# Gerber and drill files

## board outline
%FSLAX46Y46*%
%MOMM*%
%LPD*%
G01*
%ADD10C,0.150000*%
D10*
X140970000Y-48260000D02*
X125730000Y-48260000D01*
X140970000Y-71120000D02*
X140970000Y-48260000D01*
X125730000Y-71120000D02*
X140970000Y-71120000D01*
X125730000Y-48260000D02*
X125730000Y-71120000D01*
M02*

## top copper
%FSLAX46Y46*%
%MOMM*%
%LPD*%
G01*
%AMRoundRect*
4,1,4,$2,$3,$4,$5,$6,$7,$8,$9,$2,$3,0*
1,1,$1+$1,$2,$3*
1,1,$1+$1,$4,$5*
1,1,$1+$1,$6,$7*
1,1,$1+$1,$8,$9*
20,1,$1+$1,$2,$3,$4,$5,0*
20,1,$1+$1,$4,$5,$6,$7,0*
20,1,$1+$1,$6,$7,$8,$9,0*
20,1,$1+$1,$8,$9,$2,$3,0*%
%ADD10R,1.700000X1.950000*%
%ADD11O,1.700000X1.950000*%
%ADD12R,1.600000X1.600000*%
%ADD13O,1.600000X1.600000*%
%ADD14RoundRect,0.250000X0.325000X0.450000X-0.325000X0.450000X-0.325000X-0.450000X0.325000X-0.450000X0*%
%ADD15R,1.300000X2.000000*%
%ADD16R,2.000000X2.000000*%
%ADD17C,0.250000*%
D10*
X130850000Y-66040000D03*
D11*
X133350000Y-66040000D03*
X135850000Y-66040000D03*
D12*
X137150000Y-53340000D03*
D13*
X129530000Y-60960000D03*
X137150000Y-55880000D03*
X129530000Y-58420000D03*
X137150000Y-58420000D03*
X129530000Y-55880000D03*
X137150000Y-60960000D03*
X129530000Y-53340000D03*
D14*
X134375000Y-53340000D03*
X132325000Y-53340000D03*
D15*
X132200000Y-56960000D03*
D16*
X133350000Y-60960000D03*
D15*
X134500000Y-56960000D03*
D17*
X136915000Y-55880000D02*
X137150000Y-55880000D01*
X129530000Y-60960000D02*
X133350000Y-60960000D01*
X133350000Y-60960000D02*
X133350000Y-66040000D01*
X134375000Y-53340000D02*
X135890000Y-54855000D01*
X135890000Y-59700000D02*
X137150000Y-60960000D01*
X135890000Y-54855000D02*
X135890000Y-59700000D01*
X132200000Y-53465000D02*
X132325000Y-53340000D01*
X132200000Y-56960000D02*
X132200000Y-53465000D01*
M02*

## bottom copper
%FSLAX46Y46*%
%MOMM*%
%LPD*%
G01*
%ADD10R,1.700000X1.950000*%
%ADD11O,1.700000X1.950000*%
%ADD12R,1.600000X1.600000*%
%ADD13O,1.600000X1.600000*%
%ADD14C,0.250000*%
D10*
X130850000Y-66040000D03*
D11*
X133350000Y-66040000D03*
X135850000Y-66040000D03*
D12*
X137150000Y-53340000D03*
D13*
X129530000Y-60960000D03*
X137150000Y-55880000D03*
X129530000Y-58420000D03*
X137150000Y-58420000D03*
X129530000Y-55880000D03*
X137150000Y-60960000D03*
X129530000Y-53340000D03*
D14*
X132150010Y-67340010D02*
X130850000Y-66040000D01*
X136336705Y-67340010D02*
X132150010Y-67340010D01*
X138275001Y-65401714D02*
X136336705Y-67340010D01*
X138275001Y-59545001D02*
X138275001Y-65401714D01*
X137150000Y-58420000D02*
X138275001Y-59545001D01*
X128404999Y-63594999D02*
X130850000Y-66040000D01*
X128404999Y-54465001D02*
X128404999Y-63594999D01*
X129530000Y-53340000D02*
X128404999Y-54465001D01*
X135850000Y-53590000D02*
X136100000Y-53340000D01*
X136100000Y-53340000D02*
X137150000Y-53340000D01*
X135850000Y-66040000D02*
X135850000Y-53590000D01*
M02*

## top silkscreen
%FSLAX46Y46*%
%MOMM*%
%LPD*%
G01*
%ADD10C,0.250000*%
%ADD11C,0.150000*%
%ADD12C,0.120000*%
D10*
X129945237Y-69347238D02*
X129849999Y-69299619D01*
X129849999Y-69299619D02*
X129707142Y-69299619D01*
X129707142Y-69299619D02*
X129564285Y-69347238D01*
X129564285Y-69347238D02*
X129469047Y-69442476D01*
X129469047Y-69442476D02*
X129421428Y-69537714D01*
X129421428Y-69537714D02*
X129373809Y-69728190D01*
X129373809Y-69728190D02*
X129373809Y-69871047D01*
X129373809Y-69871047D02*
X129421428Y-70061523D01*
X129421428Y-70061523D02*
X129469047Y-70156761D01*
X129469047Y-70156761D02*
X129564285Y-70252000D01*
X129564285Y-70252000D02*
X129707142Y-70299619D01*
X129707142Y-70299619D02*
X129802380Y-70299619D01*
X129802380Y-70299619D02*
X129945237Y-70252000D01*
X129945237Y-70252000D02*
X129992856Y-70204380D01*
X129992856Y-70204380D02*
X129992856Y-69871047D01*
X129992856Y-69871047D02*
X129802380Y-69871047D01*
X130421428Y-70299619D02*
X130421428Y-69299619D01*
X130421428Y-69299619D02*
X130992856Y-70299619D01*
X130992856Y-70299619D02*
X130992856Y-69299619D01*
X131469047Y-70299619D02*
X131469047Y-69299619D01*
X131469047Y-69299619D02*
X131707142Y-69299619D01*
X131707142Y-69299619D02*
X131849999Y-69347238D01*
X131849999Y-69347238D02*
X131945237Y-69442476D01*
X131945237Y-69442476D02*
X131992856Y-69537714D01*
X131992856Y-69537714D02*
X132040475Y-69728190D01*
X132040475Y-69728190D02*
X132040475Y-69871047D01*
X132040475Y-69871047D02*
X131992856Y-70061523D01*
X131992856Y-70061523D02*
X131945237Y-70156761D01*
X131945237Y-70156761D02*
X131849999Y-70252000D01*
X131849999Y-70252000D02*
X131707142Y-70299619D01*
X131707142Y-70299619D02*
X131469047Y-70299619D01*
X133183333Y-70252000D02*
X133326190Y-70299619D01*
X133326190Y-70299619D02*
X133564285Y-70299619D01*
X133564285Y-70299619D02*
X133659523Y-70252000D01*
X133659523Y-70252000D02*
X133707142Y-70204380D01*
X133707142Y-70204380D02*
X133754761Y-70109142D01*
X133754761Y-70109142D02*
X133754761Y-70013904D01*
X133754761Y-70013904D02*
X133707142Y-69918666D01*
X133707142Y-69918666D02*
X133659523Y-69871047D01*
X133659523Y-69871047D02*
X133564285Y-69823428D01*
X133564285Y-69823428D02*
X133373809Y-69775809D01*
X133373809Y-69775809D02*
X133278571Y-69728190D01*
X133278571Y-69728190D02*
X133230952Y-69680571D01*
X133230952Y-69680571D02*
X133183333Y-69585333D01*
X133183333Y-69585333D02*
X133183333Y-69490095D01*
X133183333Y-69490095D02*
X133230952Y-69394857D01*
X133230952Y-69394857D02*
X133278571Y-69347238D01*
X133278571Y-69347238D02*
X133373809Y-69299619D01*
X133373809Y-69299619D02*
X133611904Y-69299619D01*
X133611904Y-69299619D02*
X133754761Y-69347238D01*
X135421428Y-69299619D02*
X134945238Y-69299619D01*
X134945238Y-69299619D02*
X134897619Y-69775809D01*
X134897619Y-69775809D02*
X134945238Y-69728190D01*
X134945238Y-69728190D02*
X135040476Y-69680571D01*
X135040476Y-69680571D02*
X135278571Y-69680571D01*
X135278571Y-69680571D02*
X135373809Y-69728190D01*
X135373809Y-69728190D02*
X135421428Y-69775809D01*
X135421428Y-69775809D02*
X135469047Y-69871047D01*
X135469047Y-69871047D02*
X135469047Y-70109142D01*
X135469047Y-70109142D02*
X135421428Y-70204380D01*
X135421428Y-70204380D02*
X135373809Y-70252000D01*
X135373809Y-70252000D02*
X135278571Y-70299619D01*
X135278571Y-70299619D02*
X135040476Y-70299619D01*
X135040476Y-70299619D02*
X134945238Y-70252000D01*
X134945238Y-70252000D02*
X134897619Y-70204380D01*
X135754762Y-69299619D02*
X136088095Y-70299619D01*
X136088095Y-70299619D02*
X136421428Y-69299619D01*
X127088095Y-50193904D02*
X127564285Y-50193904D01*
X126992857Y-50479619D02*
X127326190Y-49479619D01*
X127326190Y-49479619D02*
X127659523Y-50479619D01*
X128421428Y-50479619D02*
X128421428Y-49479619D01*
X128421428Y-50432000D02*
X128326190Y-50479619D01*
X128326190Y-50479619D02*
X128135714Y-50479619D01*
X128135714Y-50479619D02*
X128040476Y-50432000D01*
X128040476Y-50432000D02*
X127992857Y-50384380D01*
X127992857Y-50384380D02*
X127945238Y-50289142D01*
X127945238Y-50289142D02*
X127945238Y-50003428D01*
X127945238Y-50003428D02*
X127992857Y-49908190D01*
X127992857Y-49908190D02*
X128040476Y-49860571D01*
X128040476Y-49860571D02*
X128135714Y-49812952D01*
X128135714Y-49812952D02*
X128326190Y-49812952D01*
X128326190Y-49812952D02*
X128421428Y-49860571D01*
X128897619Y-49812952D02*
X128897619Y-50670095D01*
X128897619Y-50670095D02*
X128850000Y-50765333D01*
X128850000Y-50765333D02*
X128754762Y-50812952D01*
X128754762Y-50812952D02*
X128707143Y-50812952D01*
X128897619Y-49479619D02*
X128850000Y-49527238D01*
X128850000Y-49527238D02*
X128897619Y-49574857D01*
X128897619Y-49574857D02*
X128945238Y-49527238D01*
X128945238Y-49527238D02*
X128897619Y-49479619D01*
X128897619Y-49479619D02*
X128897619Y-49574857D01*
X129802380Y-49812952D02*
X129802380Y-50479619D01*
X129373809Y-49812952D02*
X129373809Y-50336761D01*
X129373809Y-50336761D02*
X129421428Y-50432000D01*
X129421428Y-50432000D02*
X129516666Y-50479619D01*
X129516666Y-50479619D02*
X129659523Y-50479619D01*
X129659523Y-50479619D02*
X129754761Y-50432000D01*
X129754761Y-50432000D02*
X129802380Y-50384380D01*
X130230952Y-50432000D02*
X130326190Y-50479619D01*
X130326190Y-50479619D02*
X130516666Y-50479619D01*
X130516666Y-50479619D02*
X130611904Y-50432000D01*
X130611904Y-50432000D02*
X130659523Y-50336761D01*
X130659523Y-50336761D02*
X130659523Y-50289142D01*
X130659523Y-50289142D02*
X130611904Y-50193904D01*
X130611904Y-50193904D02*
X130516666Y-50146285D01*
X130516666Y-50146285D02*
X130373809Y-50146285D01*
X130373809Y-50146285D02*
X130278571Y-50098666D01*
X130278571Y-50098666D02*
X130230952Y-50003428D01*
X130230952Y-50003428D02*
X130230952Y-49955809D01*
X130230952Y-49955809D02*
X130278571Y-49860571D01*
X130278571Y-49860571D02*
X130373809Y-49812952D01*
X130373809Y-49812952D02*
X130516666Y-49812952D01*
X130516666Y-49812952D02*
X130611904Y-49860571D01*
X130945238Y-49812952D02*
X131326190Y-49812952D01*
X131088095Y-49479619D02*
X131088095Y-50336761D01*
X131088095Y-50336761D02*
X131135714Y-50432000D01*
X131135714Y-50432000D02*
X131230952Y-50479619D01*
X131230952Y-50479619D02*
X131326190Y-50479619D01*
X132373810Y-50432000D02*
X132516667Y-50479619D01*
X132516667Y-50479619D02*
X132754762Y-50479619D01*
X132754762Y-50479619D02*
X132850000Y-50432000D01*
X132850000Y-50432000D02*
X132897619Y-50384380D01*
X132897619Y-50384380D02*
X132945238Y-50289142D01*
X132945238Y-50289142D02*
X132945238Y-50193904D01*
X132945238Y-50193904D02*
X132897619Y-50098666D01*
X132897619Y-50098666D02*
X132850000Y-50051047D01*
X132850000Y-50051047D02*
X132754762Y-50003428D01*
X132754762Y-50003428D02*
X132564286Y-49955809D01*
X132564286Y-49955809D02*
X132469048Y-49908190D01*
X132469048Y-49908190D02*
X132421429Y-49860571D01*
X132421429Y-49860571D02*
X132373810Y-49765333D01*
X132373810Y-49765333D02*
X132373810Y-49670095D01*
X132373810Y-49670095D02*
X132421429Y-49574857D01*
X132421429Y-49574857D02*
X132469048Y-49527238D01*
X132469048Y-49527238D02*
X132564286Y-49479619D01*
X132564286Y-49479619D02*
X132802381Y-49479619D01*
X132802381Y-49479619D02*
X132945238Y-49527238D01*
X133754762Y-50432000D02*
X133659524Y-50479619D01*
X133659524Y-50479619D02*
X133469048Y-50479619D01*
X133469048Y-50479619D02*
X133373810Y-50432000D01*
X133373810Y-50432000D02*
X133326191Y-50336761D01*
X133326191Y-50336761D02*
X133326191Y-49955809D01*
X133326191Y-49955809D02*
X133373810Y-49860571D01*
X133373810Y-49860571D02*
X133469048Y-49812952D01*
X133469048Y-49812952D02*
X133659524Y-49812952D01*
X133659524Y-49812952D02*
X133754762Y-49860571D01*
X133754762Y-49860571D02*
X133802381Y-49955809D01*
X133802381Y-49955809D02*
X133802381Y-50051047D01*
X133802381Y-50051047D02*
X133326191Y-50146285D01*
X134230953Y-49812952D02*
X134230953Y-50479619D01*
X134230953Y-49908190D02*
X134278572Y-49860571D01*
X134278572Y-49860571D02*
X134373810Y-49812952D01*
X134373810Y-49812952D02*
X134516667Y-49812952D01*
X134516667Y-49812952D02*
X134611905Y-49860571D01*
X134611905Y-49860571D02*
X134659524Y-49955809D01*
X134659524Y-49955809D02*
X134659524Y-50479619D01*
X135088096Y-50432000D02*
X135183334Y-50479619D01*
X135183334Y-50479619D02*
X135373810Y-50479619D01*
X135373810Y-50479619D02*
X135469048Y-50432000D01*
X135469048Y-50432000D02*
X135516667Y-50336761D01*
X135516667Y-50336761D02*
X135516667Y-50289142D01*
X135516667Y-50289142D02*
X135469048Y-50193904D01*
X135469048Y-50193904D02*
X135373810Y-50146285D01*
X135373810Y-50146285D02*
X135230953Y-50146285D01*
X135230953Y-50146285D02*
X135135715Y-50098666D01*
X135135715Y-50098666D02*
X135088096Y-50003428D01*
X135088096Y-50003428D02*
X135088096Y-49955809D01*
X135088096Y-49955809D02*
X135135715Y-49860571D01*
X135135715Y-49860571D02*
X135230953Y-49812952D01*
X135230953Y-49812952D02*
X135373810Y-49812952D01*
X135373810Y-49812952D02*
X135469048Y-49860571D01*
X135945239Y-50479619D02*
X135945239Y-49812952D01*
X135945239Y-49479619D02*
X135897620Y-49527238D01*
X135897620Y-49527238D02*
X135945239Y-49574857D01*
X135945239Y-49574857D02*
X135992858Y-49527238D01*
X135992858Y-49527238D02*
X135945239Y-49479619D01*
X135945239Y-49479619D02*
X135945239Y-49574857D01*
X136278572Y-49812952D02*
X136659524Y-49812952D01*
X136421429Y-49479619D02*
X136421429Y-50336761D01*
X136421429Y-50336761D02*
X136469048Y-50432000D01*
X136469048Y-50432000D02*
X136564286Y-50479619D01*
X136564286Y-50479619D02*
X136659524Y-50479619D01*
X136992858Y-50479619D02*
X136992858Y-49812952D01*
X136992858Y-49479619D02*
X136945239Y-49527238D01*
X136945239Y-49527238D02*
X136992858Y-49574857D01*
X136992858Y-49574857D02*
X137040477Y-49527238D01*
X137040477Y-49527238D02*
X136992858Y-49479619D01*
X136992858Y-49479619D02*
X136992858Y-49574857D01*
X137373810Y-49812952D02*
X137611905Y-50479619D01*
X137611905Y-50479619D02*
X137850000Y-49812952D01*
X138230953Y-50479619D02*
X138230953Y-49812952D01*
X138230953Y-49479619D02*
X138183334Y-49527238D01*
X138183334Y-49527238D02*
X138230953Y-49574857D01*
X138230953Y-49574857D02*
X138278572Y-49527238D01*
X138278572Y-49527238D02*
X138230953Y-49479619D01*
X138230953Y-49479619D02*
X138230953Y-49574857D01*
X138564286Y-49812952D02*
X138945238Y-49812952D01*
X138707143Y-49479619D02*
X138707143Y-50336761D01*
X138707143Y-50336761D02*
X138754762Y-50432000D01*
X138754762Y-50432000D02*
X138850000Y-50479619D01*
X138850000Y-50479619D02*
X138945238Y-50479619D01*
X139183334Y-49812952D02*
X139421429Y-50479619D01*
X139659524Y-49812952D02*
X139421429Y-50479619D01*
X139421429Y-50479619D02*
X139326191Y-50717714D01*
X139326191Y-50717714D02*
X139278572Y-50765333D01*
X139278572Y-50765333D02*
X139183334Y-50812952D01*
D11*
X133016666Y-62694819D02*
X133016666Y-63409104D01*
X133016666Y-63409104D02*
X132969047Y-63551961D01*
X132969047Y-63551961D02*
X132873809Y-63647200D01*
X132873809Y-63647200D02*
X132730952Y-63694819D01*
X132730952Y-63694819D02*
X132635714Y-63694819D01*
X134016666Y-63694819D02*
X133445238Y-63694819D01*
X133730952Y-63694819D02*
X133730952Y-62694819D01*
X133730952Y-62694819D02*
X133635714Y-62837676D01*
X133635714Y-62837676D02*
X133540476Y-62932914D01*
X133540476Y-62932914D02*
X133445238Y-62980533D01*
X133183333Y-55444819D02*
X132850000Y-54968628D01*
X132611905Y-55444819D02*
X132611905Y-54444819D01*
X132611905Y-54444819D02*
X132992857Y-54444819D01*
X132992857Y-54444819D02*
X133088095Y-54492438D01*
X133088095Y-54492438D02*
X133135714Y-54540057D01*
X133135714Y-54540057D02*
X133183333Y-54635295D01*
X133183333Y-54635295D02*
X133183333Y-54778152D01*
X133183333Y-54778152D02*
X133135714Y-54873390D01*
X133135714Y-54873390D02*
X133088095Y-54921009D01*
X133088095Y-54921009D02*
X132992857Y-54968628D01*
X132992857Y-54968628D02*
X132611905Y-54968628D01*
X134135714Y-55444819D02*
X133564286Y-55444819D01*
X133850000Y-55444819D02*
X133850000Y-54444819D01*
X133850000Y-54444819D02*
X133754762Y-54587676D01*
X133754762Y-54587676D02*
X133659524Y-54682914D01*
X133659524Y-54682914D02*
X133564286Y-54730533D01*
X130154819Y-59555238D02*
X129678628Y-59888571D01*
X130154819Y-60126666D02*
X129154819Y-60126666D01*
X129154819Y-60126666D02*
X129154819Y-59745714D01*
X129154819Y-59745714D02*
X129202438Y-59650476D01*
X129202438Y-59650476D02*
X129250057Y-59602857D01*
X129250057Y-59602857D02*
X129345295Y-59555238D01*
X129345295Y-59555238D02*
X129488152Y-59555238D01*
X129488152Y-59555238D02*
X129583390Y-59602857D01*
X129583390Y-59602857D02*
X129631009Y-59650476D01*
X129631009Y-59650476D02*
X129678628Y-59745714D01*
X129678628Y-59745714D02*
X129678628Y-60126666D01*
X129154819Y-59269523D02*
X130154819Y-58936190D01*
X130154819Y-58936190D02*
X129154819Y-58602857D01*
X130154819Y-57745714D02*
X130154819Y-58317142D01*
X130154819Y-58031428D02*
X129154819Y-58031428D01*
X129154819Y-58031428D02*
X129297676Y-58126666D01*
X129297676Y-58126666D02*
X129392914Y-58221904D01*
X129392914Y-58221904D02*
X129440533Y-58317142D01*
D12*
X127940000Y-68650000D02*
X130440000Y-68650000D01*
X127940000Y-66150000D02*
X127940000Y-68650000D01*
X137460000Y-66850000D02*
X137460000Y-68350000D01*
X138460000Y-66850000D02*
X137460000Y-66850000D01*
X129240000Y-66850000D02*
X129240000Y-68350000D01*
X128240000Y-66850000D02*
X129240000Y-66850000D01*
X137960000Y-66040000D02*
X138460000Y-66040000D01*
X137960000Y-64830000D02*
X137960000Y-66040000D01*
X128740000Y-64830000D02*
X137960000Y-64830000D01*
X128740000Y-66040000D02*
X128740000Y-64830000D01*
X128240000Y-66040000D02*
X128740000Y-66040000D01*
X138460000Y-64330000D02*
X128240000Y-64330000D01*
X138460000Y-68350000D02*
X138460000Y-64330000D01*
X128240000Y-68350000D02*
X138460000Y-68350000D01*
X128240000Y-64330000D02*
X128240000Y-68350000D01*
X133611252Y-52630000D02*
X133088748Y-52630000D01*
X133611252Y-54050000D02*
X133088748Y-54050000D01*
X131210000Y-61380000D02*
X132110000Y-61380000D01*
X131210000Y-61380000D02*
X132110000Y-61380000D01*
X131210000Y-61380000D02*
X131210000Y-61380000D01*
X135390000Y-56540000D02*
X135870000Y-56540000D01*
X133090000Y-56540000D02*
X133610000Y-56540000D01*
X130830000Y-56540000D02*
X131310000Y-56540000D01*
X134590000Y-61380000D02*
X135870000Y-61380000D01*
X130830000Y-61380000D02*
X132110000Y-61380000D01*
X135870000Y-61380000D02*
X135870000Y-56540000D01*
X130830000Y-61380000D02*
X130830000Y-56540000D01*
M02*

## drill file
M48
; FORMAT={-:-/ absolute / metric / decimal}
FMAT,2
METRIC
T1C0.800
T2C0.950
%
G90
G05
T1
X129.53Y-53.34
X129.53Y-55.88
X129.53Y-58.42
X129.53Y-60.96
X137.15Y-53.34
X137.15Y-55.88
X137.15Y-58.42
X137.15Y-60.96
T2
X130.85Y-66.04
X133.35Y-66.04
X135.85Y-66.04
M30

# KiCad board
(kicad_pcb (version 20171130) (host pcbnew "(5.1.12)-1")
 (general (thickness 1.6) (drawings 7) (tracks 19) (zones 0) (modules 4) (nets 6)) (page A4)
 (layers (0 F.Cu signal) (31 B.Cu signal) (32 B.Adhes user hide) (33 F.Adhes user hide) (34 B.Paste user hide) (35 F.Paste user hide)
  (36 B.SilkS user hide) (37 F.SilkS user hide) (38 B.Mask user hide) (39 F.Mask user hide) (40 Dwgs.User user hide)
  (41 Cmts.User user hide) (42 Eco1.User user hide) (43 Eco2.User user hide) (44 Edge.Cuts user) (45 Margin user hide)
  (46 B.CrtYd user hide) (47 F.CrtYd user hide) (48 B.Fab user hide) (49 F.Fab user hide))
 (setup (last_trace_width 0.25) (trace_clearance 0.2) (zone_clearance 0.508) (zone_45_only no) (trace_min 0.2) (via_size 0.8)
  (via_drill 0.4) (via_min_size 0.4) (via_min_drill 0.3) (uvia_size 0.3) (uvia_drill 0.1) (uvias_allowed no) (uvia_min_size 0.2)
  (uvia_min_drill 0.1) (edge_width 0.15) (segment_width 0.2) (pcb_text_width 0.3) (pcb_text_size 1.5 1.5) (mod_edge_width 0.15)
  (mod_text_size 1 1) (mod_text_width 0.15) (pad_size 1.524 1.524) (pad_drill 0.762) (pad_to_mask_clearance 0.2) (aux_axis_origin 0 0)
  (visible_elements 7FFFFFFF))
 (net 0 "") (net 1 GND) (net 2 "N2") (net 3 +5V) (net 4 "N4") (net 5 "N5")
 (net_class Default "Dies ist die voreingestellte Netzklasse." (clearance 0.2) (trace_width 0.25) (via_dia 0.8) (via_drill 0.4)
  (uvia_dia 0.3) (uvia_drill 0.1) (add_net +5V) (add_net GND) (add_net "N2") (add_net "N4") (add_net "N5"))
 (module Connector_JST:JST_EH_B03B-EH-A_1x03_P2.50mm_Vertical (layer F.Cu) (at 130.85 66.04)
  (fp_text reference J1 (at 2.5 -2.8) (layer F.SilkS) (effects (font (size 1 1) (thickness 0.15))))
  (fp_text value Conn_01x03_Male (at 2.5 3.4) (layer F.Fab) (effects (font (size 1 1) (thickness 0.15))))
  (fp_line (start -2.91 2.61) (end -0.41 2.61) (layer F.SilkS) (width 0.12))
  (fp_line (start -2.91 0.11) (end -2.91 2.61) (layer F.SilkS) (width 0.12))
  (fp_line (start 6.61 0.81) (end 6.61 2.31) (layer F.SilkS) (width 0.12))
  (fp_line (start 7.61 0.81) (end 6.61 0.81) (layer F.SilkS) (width 0.12))
  (fp_line (start -1.61 0.81) (end -1.61 2.31) (layer F.SilkS) (width 0.12))
  (fp_line (start -2.61 0.81) (end -1.61 0.81) (layer F.SilkS) (width 0.12))
  (fp_line (start 7.11 0) (end 7.61 0) (layer F.SilkS) (width 0.12))
  (fp_line (start 7.11 -1.21) (end 7.11 0) (layer F.SilkS) (width 0.12))
  (fp_line (start -2.11 -1.21) (end 7.11 -1.21) (layer F.SilkS) (width 0.12))
  (fp_line (start -2.11 0) (end -2.11 -1.21) (layer F.SilkS) (width 0.12))
  (fp_line (start -2.61 0) (end -2.11 0) (layer F.SilkS) (width 0.12))
  (fp_line (start 7.61 -1.71) (end -2.61 -1.71) (layer F.SilkS) (width 0.12))
  (fp_line (start 7.61 2.31) (end 7.61 -1.71) (layer F.SilkS) (width 0.12))
  (fp_line (start -2.61 2.31) (end 7.61 2.31) (layer F.SilkS) (width 0.12))
  (fp_line (start -2.61 -1.71) (end -2.61 2.31) (layer F.SilkS) (width 0.12))
  (pad 1 thru_hole rect (at 0 0) (size 1.7 1.95) (drill 0.95) (layers *.Cu *.Mask) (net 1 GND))
  (pad 2 thru_hole oval (at 2.5 0) (size 1.7 1.95) (drill 0.95) (layers *.Cu *.Mask) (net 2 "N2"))
  (pad 3 thru_hole oval (at 5 0) (size 1.7 1.95) (drill 0.95) (layers *.Cu *.Mask) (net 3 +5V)))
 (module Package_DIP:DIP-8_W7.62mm (layer B.Cu) (at 137.15 53.34 180)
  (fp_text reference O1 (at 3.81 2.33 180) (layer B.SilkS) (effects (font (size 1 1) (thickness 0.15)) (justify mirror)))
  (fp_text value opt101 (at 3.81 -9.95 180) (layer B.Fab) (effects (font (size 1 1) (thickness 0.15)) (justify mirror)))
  (pad 1 thru_hole rect (at 0 0 180) (size 1.6 1.6) (drill 0.8) (layers *.Cu *.Mask) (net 3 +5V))
  (pad 5 thru_hole oval (at 7.62 -7.62 180) (size 1.6 1.6) (drill 0.8) (layers *.Cu *.Mask) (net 2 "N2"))
  (pad 2 thru_hole oval (at 0 -2.54 180) (size 1.6 1.6) (drill 0.8) (layers *.Cu *.Mask))
  (pad 6 thru_hole oval (at 7.62 -5.08 180) (size 1.6 1.6) (drill 0.8) (layers *.Cu *.Mask))
  (pad 3 thru_hole oval (at 0 -5.08 180) (size 1.6 1.6) (drill 0.8) (layers *.Cu *.Mask) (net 1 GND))
  (pad 7 thru_hole oval (at 7.62 -2.54 180) (size 1.6 1.6) (drill 0.8) (layers *.Cu *.Mask))
  (pad 4 thru_hole oval (at 0 -7.62 180) (size 1.6 1.6) (drill 0.8) (layers *.Cu *.Mask) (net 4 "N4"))
  (pad 8 thru_hole oval (at 7.62 0 180) (size 1.6 1.6) (drill 0.8) (layers *.Cu *.Mask) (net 1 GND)))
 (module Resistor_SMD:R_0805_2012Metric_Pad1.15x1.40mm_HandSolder (layer F.Cu) (at 133.35 53.34 180)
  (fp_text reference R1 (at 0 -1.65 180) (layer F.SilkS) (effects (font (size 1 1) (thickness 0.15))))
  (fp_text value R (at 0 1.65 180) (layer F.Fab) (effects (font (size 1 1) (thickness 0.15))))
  (fp_line (start -0.261252 0.71) (end 0.261252 0.71) (layer F.SilkS) (width 0.12))
  (fp_line (start -0.261252 -0.71) (end 0.261252 -0.71) (layer F.SilkS) (width 0.12))
  (pad 1 smd roundrect (at -1.025 0 180) (size 1.15 1.4) (layers F.Cu F.Paste F.Mask) (roundrect_rratio 0.217391) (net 4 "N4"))
  (pad 2 smd roundrect (at 1.025 0 180) (size 1.15 1.4) (layers F.Cu F.Paste F.Mask) (roundrect_rratio 0.217391) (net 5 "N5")))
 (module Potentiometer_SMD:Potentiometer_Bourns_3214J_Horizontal (layer F.Cu) (at 133.35 58.96 90)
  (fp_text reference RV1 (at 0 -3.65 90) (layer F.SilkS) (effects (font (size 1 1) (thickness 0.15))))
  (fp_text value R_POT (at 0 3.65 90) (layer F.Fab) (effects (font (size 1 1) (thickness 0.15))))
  (fp_line (start -2.42 -2.14) (end -2.42 -1.24) (layer F.SilkS) (width 0.12))
  (fp_line (start -2.42 -2.14) (end -2.42 -1.24) (layer F.SilkS) (width 0.12))
  (fp_line (start -2.42 -2.14) (end -2.42 -2.14) (layer F.SilkS) (width 0.12))
  (fp_line (start 2.42 2.04) (end 2.42 2.52) (layer F.SilkS) (width 0.12))
  (fp_line (start 2.42 -0.26) (end 2.42 0.26) (layer F.SilkS) (width 0.12))
  (fp_line (start 2.42 -2.52) (end 2.42 -2.04) (layer F.SilkS) (width 0.12))
  (fp_line (start -2.42 1.24) (end -2.42 2.52) (layer F.SilkS) (width 0.12))
  (fp_line (start -2.42 -2.52) (end -2.42 -1.24) (layer F.SilkS) (width 0.12))
  (fp_line (start -2.42 2.52) (end 2.42 2.52) (layer F.SilkS) (width 0.12))
  (fp_line (start -2.42 -2.52) (end 2.42 -2.52) (layer F.SilkS) (width 0.12))
  (pad 1 smd rect (at 2 -1.15 90) (size 2 1.3) (layers F.Cu F.Paste F.Mask) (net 5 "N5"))
  (pad 2 smd rect (at -2 0 90) (size 2 2) (layers F.Cu F.Paste F.Mask) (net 2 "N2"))
  (pad 3 smd rect (at 2 1.15 90) (size 2 1.3) (layers F.Cu F.Paste F.Mask)))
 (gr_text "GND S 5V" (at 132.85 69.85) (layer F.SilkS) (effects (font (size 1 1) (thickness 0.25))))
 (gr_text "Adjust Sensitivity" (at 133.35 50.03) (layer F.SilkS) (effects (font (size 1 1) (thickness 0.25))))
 (gr_line (start 140.97 48.26) (end 125.73 48.26) (layer Edge.Cuts) (width 0.15))
 (gr_line (start 140.97 71.12) (end 140.97 48.26) (layer Edge.Cuts) (width 0.15))
 (gr_line (start 125.73 71.12) (end 140.97 71.12) (layer Edge.Cuts) (width 0.15))
 (gr_line (start 125.73 48.26) (end 125.73 71.12) (layer Edge.Cuts) (width 0.15))
 (segment (start 136.915 55.88) (end 137.15 55.88) (width 0.25) (layer F.Cu) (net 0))
 (segment (start 132.15001 67.34001) (end 130.85 66.04) (width 0.25) (layer B.Cu) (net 1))
 (segment (start 136.336705 67.34001) (end 132.15001 67.34001) (width 0.25) (layer B.Cu) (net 1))
 (segment (start 138.275001 65.401714) (end 136.336705 67.34001) (width 0.25) (layer B.Cu) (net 1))
 (segment (start 138.275001 59.545001) (end 138.275001 65.401714) (width 0.25) (layer B.Cu) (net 1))
 (segment (start 137.15 58.42) (end 138.275001 59.545001) (width 0.25) (layer B.Cu) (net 1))
 (segment (start 128.404999 63.594999) (end 130.85 66.04) (width 0.25) (layer B.Cu) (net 1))
 (segment (start 128.404999 54.465001) (end 128.404999 63.594999) (width 0.25) (layer B.Cu) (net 1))
 (segment (start 129.53 53.34) (end 128.404999 54.465001) (width 0.25) (layer B.Cu) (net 1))
 (segment (start 129.53 60.96) (end 133.35 60.96) (width 0.25) (layer F.Cu) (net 2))
 (segment (start 133.35 60.96) (end 133.35 66.04) (width 0.25) (layer F.Cu) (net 2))
 (segment (start 135.85 53.59) (end 136.1 53.34) (width 0.25) (layer B.Cu) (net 3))
 (segment (start 136.1 53.34) (end 137.15 53.34) (width 0.25) (layer B.Cu) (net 3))
 (segment (start 135.85 66.04) (end 135.85 53.59) (width 0.25) (layer B.Cu) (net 3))
 (segment (start 134.375 53.34) (end 135.89 54.855) (width 0.25) (layer F.Cu) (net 4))
 (segment (start 135.89 59.7) (end 137.15 60.96) (width 0.25) (layer F.Cu) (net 4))
 (segment (start 135.89 54.855) (end 135.89 59.7) (width 0.25) (layer F.Cu) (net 4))
 (segment (start 132.2 53.465) (end 132.325 53.34) (width 0.25) (layer F.Cu) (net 5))
 (segment (start 132.2 56.96) (end 132.2 53.465) (width 0.25) (layer F.Cu) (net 5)))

